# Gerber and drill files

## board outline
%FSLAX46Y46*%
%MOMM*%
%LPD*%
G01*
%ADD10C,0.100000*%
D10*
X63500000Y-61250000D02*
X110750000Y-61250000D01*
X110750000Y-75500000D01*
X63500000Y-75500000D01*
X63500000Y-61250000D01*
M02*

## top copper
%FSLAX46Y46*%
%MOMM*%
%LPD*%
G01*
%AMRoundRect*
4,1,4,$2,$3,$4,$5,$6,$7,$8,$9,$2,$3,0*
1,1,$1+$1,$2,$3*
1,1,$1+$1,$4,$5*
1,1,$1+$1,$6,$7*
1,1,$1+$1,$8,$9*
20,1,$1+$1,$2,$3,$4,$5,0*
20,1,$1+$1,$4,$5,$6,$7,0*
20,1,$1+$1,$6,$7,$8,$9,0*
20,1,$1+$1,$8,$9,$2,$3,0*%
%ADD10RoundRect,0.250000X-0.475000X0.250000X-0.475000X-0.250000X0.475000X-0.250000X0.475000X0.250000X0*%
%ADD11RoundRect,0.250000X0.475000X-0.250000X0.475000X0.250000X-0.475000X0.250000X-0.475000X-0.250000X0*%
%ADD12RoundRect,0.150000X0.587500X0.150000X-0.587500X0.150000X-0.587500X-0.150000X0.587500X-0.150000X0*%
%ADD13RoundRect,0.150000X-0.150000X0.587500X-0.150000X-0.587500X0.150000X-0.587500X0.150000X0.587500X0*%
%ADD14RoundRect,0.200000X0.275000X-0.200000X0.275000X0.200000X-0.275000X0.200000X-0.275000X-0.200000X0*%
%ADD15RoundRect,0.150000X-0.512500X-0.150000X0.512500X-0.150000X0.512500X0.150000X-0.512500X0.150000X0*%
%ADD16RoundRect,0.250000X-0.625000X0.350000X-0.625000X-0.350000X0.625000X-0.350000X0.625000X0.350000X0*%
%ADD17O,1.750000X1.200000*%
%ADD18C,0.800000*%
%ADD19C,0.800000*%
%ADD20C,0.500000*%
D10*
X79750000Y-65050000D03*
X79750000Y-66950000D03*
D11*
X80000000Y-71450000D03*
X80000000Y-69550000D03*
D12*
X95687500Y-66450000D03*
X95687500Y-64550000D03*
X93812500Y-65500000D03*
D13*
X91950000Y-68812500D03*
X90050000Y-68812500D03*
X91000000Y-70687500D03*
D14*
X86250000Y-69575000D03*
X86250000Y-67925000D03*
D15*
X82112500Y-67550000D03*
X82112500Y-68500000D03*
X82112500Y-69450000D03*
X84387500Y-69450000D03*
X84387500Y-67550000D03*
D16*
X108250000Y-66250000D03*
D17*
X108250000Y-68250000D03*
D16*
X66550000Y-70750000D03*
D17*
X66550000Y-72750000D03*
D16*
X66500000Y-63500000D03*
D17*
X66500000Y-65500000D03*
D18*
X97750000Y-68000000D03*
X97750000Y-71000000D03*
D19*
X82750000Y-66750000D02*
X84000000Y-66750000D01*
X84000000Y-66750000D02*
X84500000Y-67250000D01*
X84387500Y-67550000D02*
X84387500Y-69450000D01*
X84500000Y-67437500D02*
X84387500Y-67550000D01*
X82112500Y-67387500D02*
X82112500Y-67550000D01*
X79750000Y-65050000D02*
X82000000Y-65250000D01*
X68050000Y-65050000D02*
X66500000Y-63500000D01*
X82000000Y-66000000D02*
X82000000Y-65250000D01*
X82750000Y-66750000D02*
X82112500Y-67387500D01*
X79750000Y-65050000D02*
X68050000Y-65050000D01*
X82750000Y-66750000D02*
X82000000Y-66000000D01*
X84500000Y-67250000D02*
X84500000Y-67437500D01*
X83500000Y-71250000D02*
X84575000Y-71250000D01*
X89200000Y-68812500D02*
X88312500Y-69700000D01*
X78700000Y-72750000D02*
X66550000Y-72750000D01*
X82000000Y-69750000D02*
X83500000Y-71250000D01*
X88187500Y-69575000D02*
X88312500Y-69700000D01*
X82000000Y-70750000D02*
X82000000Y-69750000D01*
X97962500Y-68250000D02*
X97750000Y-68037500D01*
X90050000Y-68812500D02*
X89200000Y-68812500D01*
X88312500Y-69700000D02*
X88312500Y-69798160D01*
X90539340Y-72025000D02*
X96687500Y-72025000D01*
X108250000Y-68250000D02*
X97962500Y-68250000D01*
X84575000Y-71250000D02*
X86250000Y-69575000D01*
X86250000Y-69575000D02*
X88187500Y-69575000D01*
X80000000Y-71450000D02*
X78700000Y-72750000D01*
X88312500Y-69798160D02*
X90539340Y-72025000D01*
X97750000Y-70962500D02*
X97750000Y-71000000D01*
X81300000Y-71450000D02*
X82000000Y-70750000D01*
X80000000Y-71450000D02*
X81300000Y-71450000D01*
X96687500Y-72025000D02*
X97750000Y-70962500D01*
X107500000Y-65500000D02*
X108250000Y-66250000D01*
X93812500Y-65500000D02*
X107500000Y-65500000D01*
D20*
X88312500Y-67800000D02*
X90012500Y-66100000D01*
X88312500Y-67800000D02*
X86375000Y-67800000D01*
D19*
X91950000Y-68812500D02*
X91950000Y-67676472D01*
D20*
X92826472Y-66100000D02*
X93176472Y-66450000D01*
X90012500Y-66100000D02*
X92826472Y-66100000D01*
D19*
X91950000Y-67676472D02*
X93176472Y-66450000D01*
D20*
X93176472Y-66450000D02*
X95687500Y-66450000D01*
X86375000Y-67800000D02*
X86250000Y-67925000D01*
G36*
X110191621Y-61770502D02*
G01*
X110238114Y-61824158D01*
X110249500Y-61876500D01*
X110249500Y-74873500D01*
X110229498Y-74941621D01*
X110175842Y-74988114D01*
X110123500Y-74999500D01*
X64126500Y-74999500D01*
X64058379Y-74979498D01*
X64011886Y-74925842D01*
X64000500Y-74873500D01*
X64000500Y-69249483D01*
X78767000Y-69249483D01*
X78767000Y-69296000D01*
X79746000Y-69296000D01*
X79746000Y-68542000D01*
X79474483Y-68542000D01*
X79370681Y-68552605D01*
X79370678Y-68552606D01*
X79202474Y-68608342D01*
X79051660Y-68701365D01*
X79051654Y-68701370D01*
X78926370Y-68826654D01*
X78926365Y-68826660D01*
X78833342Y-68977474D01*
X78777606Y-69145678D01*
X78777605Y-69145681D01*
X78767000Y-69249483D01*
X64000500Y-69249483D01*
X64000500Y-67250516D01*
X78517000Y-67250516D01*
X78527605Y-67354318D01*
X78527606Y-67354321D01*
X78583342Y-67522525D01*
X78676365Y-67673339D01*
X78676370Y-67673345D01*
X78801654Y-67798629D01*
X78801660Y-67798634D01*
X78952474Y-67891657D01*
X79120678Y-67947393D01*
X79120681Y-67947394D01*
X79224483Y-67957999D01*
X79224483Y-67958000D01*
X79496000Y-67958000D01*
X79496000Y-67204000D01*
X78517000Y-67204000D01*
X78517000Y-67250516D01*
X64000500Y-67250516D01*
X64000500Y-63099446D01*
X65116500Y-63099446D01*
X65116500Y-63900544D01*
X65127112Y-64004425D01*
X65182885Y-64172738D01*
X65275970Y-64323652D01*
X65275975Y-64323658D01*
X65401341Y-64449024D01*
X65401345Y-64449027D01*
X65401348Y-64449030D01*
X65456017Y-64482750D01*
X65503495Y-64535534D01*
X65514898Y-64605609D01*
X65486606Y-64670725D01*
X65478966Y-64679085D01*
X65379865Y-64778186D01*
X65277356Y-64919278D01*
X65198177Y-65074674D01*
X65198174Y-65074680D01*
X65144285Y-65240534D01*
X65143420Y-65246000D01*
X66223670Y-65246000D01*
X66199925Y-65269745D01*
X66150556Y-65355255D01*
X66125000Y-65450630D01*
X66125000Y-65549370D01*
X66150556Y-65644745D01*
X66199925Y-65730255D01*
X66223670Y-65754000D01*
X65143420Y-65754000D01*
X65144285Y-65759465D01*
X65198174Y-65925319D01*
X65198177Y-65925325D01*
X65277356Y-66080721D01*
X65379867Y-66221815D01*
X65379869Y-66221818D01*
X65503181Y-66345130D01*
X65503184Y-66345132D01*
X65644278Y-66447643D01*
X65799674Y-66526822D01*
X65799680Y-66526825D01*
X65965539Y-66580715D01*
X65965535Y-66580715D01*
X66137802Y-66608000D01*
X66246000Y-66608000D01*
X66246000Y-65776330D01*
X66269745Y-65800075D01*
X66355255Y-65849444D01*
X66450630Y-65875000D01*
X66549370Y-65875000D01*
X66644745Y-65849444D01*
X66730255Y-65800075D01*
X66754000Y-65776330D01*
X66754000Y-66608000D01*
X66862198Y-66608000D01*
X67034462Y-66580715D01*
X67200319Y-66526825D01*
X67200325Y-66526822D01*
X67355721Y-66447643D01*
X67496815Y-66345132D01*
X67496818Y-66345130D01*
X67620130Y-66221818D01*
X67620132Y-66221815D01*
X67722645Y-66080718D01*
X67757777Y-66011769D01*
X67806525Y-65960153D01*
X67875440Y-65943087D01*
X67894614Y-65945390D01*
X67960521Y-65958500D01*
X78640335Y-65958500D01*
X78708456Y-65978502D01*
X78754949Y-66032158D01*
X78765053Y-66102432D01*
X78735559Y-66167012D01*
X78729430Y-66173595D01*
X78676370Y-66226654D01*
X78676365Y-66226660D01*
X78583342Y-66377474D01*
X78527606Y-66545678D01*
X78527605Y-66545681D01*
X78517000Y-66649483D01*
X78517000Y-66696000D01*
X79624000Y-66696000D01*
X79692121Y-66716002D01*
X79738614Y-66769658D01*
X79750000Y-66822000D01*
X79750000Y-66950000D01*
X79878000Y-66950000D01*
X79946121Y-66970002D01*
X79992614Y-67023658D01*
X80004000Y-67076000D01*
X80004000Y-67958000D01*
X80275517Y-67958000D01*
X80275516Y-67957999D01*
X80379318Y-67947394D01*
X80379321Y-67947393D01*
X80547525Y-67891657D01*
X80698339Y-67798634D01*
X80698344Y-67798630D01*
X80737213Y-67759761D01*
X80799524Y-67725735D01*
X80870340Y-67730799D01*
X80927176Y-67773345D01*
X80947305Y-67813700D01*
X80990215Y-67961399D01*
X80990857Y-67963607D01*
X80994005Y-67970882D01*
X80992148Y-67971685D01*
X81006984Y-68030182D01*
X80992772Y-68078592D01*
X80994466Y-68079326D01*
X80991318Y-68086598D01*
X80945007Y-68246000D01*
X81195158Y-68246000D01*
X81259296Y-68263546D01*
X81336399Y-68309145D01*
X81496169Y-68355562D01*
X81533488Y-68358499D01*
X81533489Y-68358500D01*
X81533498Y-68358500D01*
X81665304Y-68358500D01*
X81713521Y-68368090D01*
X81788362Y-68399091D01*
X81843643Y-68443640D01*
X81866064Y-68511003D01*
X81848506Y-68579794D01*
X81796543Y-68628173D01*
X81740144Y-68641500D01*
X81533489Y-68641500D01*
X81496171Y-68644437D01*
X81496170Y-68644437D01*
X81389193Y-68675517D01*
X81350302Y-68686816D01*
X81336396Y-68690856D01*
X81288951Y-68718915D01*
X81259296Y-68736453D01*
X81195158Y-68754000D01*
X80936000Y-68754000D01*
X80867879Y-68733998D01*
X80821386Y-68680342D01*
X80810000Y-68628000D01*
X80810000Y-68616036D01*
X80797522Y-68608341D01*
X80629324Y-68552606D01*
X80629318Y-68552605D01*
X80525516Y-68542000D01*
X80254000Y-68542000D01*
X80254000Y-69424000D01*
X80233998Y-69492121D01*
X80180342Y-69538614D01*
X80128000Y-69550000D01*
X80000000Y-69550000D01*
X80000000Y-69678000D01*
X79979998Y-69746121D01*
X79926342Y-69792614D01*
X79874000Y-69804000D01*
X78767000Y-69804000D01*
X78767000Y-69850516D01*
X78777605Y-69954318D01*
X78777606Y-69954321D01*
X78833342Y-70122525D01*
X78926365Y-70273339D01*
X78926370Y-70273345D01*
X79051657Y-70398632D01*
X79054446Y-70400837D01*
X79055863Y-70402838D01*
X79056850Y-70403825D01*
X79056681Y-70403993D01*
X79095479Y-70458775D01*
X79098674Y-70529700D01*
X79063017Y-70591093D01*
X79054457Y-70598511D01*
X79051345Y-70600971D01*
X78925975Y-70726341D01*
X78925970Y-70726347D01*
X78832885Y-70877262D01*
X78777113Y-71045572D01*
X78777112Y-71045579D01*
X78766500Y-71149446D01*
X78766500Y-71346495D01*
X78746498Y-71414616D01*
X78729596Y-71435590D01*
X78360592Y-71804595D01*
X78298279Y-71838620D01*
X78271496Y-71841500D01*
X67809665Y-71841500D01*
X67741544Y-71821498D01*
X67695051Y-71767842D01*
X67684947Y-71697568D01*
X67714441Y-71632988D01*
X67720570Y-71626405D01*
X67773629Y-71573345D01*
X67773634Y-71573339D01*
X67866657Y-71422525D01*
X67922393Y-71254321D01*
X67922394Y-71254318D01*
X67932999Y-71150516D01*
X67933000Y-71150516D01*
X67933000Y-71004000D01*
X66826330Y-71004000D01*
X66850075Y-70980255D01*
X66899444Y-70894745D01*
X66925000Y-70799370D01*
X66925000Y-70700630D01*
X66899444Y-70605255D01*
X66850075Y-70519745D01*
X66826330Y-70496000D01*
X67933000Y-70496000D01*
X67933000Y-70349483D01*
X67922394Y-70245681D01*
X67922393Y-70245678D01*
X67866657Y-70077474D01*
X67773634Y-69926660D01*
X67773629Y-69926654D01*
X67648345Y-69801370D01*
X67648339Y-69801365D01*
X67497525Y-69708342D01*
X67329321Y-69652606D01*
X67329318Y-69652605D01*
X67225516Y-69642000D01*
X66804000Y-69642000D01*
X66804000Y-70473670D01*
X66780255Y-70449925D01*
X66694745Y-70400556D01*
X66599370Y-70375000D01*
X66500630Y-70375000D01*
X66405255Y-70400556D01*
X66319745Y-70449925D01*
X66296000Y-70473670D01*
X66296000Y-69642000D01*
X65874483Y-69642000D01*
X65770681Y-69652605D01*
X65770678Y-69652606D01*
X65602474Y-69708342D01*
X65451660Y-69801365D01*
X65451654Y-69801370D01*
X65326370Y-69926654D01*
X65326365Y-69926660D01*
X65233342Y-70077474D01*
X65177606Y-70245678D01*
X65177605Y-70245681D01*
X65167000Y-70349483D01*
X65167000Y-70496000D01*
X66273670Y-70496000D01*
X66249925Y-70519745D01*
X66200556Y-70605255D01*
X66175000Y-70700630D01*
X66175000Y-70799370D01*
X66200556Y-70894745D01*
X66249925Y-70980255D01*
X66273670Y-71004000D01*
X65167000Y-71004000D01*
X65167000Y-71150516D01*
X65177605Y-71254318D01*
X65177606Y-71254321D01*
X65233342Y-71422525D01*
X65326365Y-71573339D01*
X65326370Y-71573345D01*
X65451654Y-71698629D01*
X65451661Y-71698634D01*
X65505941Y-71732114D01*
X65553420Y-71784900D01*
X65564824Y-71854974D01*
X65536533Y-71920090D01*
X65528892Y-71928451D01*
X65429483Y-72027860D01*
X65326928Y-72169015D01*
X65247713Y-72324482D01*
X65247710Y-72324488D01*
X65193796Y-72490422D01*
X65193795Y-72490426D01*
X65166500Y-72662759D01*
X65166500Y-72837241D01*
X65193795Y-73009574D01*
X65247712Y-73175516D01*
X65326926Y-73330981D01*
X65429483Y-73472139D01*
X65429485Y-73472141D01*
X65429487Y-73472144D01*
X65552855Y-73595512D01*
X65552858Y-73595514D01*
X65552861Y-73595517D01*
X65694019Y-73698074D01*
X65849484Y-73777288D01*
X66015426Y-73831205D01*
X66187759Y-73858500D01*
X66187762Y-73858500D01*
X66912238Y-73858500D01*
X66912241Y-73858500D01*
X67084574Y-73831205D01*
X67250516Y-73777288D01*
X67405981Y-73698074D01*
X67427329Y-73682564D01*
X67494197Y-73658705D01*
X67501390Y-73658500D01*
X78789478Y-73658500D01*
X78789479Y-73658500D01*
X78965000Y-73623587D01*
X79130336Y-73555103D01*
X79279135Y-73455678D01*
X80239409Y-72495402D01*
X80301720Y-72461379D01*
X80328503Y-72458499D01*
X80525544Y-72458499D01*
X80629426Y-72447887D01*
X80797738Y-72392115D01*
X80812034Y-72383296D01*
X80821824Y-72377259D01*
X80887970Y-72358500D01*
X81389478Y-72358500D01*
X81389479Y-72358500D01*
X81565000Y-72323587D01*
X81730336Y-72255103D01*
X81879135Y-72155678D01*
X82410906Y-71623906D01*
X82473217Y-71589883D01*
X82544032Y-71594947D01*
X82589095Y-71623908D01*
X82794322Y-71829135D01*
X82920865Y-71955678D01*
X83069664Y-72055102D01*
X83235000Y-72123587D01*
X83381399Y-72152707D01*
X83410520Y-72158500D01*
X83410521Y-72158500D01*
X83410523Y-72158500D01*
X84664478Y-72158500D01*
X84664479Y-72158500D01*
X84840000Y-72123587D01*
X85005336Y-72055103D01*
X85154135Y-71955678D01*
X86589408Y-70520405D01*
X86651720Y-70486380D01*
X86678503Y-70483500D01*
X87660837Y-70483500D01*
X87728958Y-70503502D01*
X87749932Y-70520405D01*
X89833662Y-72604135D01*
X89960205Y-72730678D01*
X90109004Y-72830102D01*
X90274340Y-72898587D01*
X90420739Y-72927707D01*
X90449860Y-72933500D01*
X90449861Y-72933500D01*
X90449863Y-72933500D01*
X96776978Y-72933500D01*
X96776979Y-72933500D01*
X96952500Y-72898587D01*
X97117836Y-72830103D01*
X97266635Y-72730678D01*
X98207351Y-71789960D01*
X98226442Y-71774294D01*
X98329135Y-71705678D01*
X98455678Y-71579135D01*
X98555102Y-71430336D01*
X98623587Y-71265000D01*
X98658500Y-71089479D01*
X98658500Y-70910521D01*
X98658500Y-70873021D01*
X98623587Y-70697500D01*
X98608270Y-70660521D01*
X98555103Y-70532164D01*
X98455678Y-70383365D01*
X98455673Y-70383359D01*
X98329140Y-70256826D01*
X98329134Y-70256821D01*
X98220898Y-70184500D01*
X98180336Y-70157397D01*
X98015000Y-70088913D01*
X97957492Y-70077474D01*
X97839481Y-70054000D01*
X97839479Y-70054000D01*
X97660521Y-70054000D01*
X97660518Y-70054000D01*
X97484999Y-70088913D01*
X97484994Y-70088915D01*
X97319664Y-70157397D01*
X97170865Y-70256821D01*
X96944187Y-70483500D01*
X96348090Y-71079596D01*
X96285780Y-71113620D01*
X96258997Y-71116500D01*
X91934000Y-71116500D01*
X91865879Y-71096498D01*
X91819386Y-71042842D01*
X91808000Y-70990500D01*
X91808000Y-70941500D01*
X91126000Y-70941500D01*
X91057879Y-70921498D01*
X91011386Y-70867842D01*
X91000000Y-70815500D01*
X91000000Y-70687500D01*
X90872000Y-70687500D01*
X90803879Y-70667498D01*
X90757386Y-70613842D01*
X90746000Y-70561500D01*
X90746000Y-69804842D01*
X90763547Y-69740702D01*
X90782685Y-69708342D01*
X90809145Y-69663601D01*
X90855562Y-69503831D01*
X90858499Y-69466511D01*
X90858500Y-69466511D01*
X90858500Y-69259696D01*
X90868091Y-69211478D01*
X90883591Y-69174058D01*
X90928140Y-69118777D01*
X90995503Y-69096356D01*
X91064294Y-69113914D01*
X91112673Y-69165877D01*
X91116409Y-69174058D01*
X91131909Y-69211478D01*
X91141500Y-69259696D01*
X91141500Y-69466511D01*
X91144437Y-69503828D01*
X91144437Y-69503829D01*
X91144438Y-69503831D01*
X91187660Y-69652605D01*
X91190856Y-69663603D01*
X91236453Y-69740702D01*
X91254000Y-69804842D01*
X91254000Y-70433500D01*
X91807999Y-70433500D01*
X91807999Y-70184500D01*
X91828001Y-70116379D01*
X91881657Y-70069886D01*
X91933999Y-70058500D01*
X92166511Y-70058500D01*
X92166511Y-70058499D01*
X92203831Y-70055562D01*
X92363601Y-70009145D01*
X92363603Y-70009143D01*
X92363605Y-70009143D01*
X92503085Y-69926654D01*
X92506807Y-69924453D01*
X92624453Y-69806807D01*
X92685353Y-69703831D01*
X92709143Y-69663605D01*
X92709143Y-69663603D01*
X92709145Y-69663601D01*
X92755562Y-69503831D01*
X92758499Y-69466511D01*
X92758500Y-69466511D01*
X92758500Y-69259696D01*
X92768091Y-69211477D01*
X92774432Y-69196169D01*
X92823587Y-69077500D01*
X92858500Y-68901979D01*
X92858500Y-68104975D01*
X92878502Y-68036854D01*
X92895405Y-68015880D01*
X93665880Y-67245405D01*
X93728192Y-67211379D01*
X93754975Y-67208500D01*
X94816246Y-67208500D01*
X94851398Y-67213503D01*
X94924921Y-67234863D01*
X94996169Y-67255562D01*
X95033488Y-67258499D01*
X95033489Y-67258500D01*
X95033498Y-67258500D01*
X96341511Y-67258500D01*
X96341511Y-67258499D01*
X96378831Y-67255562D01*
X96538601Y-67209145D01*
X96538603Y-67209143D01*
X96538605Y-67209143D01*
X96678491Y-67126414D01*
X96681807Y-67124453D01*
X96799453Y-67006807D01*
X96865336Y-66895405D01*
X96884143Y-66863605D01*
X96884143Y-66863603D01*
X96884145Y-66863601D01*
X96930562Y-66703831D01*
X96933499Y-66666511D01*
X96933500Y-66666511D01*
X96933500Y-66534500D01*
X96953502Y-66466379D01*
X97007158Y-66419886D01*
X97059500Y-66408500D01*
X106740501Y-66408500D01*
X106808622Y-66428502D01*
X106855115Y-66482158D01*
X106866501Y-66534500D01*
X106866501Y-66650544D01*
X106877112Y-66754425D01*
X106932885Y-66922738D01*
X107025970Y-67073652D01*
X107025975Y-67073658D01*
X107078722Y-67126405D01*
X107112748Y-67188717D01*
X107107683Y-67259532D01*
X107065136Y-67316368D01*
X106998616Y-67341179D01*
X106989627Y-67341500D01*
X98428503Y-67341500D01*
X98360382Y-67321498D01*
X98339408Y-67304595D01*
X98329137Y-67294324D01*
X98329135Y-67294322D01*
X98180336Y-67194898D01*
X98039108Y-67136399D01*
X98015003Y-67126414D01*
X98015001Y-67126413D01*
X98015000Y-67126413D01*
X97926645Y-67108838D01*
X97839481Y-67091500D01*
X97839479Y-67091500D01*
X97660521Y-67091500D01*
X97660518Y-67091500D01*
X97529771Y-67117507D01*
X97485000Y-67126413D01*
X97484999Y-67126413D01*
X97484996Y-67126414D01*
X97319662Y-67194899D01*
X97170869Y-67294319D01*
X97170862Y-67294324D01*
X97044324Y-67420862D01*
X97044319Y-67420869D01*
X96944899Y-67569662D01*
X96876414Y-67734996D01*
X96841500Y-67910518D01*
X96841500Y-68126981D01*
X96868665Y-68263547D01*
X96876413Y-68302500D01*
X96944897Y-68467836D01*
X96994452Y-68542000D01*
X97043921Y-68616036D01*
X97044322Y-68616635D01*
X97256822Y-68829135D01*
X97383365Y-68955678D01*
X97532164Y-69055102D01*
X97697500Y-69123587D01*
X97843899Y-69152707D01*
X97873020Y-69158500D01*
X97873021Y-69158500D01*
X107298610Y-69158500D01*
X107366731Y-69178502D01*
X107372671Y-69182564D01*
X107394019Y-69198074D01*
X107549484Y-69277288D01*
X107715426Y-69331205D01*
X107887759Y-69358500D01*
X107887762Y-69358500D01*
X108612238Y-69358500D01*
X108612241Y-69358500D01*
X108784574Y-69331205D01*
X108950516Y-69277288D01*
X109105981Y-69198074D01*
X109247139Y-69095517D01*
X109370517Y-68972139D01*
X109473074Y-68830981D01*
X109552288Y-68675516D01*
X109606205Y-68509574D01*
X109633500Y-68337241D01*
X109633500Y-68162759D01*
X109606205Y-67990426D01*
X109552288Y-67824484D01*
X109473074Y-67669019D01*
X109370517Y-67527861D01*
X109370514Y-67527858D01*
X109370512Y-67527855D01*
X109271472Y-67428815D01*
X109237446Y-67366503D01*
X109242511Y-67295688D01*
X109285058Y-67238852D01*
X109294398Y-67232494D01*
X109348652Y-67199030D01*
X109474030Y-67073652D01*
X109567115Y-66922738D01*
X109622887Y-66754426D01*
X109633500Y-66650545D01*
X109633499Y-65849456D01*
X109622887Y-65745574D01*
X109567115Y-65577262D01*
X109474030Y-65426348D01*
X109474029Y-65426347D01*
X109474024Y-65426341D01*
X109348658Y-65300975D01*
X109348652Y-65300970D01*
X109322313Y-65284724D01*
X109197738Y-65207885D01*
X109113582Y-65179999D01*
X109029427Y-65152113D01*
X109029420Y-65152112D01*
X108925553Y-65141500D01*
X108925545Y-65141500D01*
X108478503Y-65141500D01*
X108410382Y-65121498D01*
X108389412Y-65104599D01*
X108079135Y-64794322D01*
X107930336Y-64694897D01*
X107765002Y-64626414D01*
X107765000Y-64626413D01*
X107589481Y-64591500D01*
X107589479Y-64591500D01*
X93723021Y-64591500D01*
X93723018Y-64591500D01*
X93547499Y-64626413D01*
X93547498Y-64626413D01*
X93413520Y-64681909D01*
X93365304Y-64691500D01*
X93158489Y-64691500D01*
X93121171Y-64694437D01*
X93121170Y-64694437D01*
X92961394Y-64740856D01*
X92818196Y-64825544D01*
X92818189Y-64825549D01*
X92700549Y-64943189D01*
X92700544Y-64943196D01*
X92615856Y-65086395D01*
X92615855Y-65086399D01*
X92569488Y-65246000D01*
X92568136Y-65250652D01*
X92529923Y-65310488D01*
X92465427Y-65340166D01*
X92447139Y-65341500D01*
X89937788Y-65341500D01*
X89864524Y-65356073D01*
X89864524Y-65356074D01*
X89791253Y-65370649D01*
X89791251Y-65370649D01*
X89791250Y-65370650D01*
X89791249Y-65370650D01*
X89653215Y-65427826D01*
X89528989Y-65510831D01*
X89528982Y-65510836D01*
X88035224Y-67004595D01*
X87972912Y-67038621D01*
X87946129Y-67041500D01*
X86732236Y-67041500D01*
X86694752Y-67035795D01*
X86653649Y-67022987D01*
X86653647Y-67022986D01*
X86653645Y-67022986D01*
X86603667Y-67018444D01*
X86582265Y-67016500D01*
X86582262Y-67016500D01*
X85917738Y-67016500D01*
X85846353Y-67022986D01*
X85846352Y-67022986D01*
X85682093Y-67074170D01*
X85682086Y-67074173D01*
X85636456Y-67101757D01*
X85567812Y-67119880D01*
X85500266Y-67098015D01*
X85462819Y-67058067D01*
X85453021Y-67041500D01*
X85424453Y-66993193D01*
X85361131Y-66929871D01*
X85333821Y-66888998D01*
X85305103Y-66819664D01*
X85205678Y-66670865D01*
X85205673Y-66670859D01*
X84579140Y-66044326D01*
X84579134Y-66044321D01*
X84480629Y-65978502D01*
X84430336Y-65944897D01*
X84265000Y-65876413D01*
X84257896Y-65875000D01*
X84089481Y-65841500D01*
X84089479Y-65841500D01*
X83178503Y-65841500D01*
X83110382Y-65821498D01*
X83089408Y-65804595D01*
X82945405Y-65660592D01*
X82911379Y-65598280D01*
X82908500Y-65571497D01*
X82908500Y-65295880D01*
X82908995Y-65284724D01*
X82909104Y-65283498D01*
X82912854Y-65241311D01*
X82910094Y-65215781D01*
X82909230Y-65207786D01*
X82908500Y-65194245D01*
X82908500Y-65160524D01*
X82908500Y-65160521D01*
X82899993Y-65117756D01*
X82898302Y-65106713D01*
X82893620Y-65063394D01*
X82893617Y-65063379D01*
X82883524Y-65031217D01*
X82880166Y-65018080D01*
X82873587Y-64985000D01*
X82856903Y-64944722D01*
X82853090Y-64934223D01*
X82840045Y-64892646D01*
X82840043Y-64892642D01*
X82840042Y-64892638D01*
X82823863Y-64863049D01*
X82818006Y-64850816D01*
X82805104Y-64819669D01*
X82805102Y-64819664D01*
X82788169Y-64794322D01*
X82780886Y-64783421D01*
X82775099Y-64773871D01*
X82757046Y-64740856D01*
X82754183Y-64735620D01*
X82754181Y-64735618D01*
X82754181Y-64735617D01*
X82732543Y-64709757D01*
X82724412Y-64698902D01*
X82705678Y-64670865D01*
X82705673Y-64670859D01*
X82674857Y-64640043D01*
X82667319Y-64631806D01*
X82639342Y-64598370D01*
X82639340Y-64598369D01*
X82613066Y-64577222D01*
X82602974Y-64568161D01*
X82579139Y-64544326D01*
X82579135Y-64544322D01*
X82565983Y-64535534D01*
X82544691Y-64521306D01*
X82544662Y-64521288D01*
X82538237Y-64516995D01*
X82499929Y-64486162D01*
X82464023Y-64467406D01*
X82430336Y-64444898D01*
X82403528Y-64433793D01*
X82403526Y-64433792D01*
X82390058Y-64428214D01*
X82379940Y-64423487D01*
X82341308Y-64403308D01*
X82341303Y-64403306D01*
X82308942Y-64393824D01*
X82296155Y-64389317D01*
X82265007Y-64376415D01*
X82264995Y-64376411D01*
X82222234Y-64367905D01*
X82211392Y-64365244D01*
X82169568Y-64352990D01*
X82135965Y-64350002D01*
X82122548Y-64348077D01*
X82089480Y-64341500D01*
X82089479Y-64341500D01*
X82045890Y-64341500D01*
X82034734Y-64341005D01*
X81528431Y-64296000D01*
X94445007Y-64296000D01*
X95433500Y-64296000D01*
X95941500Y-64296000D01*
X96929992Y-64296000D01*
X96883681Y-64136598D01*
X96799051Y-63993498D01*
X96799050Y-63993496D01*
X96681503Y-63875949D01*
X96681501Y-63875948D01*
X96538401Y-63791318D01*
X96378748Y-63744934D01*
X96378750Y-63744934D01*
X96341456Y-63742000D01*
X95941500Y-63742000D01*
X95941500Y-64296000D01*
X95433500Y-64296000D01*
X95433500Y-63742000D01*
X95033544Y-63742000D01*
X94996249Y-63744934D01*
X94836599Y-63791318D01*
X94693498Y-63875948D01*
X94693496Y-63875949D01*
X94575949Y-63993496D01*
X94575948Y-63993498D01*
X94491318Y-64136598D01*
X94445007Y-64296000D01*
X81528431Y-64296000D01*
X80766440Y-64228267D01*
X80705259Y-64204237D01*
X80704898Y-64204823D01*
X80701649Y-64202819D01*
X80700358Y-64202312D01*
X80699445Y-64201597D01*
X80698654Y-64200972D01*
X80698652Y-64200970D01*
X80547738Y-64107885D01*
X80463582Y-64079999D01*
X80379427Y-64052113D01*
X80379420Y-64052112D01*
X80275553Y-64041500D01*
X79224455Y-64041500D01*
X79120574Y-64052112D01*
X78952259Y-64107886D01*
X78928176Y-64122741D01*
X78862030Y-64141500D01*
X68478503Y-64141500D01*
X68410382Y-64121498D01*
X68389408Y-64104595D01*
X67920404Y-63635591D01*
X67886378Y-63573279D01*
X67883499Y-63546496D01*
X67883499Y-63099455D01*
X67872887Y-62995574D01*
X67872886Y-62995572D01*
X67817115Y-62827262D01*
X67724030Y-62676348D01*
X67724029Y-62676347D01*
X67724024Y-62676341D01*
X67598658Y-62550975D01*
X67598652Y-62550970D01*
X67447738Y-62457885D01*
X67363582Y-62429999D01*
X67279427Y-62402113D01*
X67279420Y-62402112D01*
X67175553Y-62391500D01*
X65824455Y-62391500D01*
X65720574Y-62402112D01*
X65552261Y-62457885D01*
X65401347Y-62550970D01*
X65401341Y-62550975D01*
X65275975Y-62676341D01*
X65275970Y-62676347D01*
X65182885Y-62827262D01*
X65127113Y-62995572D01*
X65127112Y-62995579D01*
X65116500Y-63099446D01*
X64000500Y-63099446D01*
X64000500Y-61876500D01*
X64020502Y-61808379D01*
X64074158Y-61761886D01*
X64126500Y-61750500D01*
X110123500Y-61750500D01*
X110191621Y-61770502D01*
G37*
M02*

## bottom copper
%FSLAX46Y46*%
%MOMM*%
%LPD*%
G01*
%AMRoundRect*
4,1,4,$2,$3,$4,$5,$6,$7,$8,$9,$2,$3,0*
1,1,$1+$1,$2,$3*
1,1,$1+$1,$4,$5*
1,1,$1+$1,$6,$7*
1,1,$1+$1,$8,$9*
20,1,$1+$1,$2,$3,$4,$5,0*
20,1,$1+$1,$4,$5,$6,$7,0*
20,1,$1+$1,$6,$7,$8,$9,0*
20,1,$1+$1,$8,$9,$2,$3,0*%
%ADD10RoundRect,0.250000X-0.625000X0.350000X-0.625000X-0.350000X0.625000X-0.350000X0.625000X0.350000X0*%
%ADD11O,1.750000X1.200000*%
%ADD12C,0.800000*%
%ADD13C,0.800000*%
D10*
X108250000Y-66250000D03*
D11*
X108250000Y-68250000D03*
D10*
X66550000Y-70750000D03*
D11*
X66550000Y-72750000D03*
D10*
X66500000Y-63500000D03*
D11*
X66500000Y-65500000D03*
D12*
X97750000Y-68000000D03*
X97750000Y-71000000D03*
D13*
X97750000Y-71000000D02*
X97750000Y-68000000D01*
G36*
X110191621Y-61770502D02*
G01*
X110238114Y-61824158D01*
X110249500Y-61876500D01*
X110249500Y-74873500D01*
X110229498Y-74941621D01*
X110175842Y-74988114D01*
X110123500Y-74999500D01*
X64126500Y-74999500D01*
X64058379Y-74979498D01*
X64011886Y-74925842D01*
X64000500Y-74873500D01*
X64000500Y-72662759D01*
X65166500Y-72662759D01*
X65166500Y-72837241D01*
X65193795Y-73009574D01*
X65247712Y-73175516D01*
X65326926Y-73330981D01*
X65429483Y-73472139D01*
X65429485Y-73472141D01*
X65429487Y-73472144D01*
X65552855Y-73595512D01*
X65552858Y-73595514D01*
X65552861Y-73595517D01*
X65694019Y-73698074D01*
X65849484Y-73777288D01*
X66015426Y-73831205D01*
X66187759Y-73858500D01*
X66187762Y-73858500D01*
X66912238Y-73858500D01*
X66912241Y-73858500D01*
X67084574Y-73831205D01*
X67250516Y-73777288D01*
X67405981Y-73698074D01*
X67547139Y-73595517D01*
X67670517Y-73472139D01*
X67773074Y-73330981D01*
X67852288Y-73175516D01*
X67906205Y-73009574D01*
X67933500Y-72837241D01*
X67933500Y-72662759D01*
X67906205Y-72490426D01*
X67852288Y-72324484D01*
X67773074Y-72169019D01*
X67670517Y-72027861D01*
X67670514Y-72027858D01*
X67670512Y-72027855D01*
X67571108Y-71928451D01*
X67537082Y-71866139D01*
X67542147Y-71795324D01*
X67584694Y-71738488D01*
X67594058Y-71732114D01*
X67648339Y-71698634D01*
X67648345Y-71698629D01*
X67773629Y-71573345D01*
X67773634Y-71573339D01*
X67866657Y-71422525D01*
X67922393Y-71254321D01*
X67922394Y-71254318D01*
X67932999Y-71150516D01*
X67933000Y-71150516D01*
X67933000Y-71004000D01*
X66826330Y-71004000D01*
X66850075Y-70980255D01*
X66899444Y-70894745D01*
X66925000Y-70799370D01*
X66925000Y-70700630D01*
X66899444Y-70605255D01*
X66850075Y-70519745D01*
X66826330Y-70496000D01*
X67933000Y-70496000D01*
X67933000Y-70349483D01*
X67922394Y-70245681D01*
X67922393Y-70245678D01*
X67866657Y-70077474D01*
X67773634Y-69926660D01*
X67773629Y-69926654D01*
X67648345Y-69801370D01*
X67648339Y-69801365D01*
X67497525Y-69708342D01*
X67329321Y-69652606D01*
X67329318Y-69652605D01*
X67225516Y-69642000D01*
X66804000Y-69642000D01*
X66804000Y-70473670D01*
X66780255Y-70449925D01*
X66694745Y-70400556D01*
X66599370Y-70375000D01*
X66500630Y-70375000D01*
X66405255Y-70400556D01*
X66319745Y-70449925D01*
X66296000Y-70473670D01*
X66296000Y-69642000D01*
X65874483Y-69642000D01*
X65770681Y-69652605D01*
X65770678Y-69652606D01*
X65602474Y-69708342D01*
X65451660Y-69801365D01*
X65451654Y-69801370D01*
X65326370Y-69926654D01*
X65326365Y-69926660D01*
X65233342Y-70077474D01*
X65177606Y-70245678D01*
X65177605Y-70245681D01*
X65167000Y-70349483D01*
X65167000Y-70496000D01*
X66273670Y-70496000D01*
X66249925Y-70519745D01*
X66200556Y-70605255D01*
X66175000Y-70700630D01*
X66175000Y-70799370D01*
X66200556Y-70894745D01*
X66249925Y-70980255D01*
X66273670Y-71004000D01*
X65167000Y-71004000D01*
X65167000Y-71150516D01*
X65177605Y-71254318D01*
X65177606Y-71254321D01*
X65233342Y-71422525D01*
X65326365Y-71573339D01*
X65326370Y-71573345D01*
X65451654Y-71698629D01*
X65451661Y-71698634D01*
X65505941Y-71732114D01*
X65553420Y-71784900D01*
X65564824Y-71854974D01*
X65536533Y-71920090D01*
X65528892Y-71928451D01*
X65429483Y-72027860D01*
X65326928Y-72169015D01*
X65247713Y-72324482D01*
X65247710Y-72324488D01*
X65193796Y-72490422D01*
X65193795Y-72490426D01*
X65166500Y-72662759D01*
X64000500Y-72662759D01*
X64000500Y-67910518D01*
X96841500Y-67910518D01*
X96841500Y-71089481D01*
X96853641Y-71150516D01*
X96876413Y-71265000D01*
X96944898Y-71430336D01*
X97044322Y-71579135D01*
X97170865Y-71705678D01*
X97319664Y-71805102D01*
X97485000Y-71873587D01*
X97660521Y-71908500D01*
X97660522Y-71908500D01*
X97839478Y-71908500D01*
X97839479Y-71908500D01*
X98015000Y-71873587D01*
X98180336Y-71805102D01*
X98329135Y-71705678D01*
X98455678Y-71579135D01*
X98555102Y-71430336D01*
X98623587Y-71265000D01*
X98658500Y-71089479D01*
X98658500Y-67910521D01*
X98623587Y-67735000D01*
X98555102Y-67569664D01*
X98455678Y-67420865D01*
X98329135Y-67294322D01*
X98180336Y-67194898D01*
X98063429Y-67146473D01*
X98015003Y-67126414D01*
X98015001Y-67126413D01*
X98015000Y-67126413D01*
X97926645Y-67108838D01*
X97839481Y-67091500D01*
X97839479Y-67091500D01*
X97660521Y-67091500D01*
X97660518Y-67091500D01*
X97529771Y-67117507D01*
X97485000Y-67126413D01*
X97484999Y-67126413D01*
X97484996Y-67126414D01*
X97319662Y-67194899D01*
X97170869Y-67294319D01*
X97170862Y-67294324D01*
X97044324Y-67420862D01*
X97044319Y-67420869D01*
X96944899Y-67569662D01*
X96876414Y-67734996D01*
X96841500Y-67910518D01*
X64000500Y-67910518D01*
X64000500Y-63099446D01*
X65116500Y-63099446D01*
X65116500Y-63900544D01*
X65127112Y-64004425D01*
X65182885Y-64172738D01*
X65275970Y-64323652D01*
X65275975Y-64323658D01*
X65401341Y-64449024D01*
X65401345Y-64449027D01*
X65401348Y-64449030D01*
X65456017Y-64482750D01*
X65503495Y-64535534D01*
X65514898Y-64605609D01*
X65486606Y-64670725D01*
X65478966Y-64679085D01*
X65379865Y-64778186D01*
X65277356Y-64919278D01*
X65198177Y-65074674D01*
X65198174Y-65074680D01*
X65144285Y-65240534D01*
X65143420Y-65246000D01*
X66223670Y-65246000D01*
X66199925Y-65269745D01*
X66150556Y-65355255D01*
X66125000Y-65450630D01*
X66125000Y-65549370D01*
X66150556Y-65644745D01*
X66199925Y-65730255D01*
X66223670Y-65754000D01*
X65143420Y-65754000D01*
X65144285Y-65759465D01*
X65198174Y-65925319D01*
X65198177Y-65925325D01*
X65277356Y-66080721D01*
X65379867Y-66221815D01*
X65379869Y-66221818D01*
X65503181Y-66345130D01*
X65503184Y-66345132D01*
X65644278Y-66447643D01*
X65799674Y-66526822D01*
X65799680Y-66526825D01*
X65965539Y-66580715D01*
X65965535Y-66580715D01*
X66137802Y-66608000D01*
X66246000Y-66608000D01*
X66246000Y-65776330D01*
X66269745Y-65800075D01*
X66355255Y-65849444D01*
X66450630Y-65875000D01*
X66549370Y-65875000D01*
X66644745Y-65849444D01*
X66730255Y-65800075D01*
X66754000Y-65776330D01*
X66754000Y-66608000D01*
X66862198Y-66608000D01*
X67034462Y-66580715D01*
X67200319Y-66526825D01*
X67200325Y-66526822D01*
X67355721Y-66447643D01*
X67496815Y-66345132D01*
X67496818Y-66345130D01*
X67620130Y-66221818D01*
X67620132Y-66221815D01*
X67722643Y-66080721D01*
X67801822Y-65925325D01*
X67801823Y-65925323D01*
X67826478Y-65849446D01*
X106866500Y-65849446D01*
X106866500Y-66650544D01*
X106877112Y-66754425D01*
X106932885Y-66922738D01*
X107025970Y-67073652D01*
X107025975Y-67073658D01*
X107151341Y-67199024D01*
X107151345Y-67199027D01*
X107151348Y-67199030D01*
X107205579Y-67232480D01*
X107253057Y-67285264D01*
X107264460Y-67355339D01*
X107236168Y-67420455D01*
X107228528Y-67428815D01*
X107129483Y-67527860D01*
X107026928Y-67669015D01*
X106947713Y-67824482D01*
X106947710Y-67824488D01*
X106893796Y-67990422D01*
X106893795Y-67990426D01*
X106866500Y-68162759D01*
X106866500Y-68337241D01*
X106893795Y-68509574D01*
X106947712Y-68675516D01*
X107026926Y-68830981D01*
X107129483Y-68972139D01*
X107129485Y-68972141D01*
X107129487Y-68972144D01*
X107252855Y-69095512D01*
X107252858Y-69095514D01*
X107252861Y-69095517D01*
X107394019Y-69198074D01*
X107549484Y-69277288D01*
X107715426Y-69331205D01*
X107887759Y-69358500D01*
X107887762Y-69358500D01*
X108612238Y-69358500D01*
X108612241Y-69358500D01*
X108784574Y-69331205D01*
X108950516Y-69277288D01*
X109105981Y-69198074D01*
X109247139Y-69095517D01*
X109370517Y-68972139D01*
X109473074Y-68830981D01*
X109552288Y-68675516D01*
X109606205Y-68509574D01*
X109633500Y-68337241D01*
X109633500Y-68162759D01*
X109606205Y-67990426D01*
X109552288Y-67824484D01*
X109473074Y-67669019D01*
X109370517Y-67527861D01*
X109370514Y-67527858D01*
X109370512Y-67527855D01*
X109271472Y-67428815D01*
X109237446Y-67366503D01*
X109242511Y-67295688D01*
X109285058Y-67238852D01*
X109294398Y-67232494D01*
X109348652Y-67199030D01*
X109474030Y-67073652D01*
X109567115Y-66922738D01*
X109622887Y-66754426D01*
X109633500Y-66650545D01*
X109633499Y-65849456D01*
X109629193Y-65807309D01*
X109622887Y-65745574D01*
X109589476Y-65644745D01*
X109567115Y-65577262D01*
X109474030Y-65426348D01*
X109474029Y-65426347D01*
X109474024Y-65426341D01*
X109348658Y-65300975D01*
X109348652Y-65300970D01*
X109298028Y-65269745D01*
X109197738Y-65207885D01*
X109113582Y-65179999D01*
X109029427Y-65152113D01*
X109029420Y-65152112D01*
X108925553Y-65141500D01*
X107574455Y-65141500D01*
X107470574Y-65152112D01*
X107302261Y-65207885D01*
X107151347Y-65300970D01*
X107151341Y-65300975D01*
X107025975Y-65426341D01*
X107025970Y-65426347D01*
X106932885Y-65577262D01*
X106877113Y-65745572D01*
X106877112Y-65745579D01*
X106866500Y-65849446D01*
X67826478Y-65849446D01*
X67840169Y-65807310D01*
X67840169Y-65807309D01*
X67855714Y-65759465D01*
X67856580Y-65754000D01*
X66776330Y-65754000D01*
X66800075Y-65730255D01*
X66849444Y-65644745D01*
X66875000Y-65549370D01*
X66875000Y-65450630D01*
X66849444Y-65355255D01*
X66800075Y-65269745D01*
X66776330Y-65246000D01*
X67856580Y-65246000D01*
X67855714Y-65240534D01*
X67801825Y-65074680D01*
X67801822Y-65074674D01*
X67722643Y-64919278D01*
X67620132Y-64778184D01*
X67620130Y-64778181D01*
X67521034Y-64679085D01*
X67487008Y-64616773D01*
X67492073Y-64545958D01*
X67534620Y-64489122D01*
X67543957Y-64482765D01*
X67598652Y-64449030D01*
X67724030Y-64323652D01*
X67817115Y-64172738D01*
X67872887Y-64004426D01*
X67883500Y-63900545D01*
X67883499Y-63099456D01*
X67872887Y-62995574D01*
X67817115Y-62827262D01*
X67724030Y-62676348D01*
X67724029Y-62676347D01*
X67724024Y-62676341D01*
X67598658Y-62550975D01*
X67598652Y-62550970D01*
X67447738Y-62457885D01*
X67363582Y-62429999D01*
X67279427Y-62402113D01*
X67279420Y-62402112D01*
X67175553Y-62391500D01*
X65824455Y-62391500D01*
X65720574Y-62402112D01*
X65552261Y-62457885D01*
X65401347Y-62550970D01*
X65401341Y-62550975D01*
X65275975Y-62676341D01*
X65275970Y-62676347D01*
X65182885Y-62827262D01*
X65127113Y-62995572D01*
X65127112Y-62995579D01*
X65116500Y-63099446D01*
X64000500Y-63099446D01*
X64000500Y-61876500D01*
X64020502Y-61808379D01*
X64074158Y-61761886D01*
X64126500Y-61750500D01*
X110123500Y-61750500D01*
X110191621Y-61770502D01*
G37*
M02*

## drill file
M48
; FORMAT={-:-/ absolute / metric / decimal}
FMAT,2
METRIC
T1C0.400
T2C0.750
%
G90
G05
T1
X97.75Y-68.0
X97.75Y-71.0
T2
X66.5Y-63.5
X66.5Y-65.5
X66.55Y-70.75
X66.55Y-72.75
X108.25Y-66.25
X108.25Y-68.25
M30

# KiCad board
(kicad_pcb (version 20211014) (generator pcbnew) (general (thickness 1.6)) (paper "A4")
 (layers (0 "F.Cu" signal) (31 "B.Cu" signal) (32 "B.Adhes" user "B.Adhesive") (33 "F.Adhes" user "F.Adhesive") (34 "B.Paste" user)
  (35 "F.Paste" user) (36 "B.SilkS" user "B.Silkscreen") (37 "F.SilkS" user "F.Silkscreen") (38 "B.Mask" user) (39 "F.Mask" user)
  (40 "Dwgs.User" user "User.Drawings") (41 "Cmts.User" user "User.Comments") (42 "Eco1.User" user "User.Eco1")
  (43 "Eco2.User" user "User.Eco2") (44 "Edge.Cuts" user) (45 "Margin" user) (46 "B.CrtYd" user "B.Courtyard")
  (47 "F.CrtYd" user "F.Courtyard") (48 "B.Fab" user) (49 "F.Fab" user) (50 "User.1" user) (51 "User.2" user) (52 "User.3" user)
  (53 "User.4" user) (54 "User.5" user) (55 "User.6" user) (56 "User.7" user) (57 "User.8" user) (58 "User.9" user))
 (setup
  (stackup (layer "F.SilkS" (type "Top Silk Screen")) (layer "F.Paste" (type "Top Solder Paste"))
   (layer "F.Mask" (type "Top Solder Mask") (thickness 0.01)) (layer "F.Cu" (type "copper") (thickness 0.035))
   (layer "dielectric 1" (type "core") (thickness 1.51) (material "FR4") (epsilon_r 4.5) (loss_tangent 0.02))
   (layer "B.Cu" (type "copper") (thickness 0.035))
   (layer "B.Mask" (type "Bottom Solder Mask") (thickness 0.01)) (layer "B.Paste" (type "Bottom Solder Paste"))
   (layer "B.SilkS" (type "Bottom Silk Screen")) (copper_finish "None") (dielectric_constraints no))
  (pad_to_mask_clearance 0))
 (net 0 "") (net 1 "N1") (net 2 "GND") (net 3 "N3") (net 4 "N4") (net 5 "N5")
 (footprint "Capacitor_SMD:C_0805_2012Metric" (layer "F.Cu") (at 79.75 66 -90)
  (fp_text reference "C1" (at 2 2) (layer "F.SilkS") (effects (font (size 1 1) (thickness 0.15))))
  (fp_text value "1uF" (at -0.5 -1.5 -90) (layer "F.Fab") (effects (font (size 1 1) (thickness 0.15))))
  (pad "1" smd roundrect (at -0.95 0 270) (size 1 1.45) (layers "F.Cu" "F.Paste" "F.Mask") (roundrect_rratio 0.25) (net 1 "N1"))
  (pad "2" smd roundrect (at 0.95 0 270) (size 1 1.45) (layers "F.Cu" "F.Paste" "F.Mask") (roundrect_rratio 0.25) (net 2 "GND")))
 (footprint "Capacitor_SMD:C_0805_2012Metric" (layer "F.Cu") (at 80 70.5 90)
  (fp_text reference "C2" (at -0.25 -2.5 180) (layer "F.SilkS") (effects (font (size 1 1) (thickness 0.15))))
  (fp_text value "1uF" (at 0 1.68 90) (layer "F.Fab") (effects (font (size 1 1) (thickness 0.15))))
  (pad "1" smd roundrect (at -0.95 0 90) (size 1 1.45) (layers "F.Cu" "F.Paste" "F.Mask") (roundrect_rratio 0.25) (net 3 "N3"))
  (pad "2" smd roundrect (at 0.95 0 90) (size 1 1.45) (layers "F.Cu" "F.Paste" "F.Mask") (roundrect_rratio 0.25) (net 2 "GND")))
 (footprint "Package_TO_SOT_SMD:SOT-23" (layer "F.Cu") (at 94.75 65.5 180)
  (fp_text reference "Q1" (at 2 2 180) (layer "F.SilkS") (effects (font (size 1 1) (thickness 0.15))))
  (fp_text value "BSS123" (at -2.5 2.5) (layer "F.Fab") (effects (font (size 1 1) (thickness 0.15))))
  (pad "1" smd roundrect (at -0.9375 -0.95 180) (size 1.475 0.6) (layers "F.Cu" "F.Paste" "F.Mask") (roundrect_rratio 0.25) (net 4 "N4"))
  (pad "2" smd roundrect (at -0.9375 0.95 180) (size 1.475 0.6) (layers "F.Cu" "F.Paste" "F.Mask") (roundrect_rratio 0.25) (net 2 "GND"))
  (pad "3" smd roundrect (at 0.9375 0 180) (size 1.475 0.6) (layers "F.Cu" "F.Paste" "F.Mask") (roundrect_rratio 0.25) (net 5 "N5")))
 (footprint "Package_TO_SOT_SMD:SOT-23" (layer "F.Cu") (at 91 69.75 -90)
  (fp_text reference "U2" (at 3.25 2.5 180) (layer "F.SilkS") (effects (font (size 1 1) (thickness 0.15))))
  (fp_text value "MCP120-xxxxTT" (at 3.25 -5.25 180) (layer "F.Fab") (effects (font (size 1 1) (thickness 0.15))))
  (pad "1" smd roundrect (at -0.9375 -0.95 270) (size 1.475 0.6) (layers "F.Cu" "F.Paste" "F.Mask") (roundrect_rratio 0.25) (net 4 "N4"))
  (pad "2" smd roundrect (at -0.9375 0.95 270) (size 1.475 0.6) (layers "F.Cu" "F.Paste" "F.Mask") (roundrect_rratio 0.25) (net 3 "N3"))
  (pad "3" smd roundrect (at 0.9375 0 270) (size 1.475 0.6) (layers "F.Cu" "F.Paste" "F.Mask") (roundrect_rratio 0.25) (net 2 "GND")))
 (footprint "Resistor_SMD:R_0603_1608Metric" (layer "F.Cu") (at 86.25 68.75 90)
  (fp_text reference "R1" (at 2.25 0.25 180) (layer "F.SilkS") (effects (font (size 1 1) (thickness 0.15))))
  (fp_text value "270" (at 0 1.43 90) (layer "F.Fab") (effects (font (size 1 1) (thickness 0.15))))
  (pad "1" smd roundrect (at -0.825 0 90) (size 0.8 0.95) (layers "F.Cu" "F.Paste" "F.Mask") (roundrect_rratio 0.25) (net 3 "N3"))
  (pad "2" smd roundrect (at 0.825 0 90) (size 0.8 0.95) (layers "F.Cu" "F.Paste" "F.Mask") (roundrect_rratio 0.25) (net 4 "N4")))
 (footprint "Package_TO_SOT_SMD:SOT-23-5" (layer "F.Cu") (at 83.25 68.5)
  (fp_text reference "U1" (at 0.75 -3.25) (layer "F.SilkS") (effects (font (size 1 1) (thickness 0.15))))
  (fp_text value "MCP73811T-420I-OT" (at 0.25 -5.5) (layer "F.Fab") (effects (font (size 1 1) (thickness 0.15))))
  (pad "1" smd roundrect (at -1.1375 -0.95) (size 1.325 0.6) (layers "F.Cu" "F.Paste" "F.Mask") (roundrect_rratio 0.25) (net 1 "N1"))
  (pad "2" smd roundrect (at -1.1375 0) (size 1.325 0.6) (layers "F.Cu" "F.Paste" "F.Mask") (roundrect_rratio 0.25) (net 2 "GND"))
  (pad "3" smd roundrect (at -1.1375 0.95) (size 1.325 0.6) (layers "F.Cu" "F.Paste" "F.Mask") (roundrect_rratio 0.25) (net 3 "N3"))
  (pad "4" smd roundrect (at 1.1375 0.95) (size 1.325 0.6) (layers "F.Cu" "F.Paste" "F.Mask") (roundrect_rratio 0.25) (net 1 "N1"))
  (pad "5" smd roundrect (at 1.1375 -0.95) (size 1.325 0.6) (layers "F.Cu" "F.Paste" "F.Mask") (roundrect_rratio 0.25) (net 1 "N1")))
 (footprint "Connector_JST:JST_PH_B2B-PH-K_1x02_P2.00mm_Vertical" (layer "B.Cu") (at 108.25 66.25 -90)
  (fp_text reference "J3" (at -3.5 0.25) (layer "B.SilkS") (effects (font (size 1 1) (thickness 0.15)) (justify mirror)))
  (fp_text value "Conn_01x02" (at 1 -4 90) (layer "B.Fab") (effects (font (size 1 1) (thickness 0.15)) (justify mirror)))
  (pad "1" thru_hole roundrect (at 0 0 270) (size 1.2 1.75) (drill 0.75) (layers *.Cu *.Mask) (roundrect_rratio 0.2083333333) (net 5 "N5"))
  (pad "2" thru_hole oval (at 2 0 270) (size 1.2 1.75) (drill 0.75) (layers *.Cu *.Mask) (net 3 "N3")))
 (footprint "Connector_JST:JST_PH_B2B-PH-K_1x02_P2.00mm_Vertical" (layer "B.Cu") (at 66.55 70.75 -90)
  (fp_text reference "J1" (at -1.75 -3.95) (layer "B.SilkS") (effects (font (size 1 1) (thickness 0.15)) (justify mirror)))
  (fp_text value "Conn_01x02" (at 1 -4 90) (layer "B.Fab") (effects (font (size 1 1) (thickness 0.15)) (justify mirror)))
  (pad "1" thru_hole roundrect (at 0 0 270) (size 1.2 1.75) (drill 0.75) (layers *.Cu *.Mask) (roundrect_rratio 0.2083333333) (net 2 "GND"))
  (pad "2" thru_hole oval (at 2 0 270) (size 1.2 1.75) (drill 0.75) (layers *.Cu *.Mask) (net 3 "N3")))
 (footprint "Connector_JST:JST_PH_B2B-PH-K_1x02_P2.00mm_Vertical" (layer "B.Cu") (at 66.5 63.5 -90)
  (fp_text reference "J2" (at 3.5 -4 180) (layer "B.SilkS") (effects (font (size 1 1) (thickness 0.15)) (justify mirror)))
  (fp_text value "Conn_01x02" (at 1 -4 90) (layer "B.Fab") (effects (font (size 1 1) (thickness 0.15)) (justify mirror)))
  (pad "1" thru_hole roundrect (at 0 0 270) (size 1.2 1.75) (drill 0.75) (layers *.Cu *.Mask) (roundrect_rratio 0.2083333333) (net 1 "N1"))
  (pad "2" thru_hole oval (at 2 0 270) (size 1.2 1.75) (drill 0.75) (layers *.Cu *.Mask) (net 2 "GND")))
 (gr_rect (start 63.5 61.25) (end 110.75 75.5) (layer "Edge.Cuts") (width 0.1) (fill none))
 (segment (start 82.75 66.75) (end 84 66.75) (width 0.8) (layer "F.Cu") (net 1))
 (segment (start 84 66.75) (end 84.5 67.25) (width 0.8) (layer "F.Cu") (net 1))
 (segment (start 84.3875 67.55) (end 84.3875 69.45) (width 0.8) (layer "F.Cu") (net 1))
 (segment (start 84.5 67.4375) (end 84.3875 67.55) (width 0.8) (layer "F.Cu") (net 1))
 (segment (start 82.1125 67.3875) (end 82.1125 67.55) (width 0.8) (layer "F.Cu") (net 1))
 (segment (start 79.75 65.05) (end 82 65.25) (width 0.8) (layer "F.Cu") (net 1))
 (segment (start 68.05 65.05) (end 66.5 63.5) (width 0.8) (layer "F.Cu") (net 1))
 (segment (start 82 66) (end 82 65.25) (width 0.8) (layer "F.Cu") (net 1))
 (segment (start 82.75 66.75) (end 82.1125 67.3875) (width 0.8) (layer "F.Cu") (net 1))
 (segment (start 79.75 65.05) (end 68.05 65.05) (width 0.8) (layer "F.Cu") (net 1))
 (segment (start 82.75 66.75) (end 82 66) (width 0.8) (layer "F.Cu") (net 1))
 (segment (start 84.5 67.25) (end 84.5 67.4375) (width 0.8) (layer "F.Cu") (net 1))
 (segment (start 83.5 71.25) (end 84.575 71.25) (width 0.8) (layer "F.Cu") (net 3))
 (segment (start 89.2 68.8125) (end 88.3125 69.7) (width 0.8) (layer "F.Cu") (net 3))
 (segment (start 78.7 72.75) (end 66.55 72.75) (width 0.8) (layer "F.Cu") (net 3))
 (segment (start 82 69.75) (end 83.5 71.25) (width 0.8) (layer "F.Cu") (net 3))
 (segment (start 88.1875 69.575) (end 88.3125 69.7) (width 0.8) (layer "F.Cu") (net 3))
 (segment (start 82 70.75) (end 82 69.75) (width 0.8) (layer "F.Cu") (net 3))
 (segment (start 97.9625 68.25) (end 97.75 68.0375) (width 0.8) (layer "F.Cu") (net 3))
 (segment (start 90.05 68.8125) (end 89.2 68.8125) (width 0.8) (layer "F.Cu") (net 3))
 (segment (start 88.3125 69.7) (end 88.3125 69.79816) (width 0.8) (layer "F.Cu") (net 3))
 (segment (start 90.53934 72.025) (end 96.6875 72.025) (width 0.8) (layer "F.Cu") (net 3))
 (segment (start 108.25 68.25) (end 97.9625 68.25) (width 0.8) (layer "F.Cu") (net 3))
 (segment (start 84.575 71.25) (end 86.25 69.575) (width 0.8) (layer "F.Cu") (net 3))
 (segment (start 86.25 69.575) (end 88.1875 69.575) (width 0.8) (layer "F.Cu") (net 3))
 (segment (start 80 71.45) (end 78.7 72.75) (width 0.8) (layer "F.Cu") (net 3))
 (segment (start 88.3125 69.79816) (end 90.53934 72.025) (width 0.8) (layer "F.Cu") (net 3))
 (segment (start 97.75 70.9625) (end 97.75 71) (width 0.8) (layer "F.Cu") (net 3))
 (segment (start 81.3 71.45) (end 82 70.75) (width 0.8) (layer "F.Cu") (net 3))
 (segment (start 80 71.45) (end 81.3 71.45) (width 0.8) (layer "F.Cu") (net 3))
 (segment (start 96.6875 72.025) (end 97.75 70.9625) (width 0.8) (layer "F.Cu") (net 3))
 (via (at 97.75 68) (size 0.8) (drill 0.4) (layers "F.Cu" "B.Cu") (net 3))
 (via (at 97.75 71) (size 0.8) (drill 0.4) (layers "F.Cu" "B.Cu") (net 3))
 (segment (start 97.75 71) (end 97.75 68) (width 0.8) (layer "B.Cu") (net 3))
 (segment (start 107.5 65.5) (end 108.25 66.25) (width 0.8) (layer "F.Cu") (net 5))
 (segment (start 93.8125 65.5) (end 107.5 65.5) (width 0.8) (layer "F.Cu") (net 5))
 (segment (start 88.3125 67.8) (end 90.0125 66.1) (width 0.5) (layer "F.Cu") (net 4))
 (segment (start 88.3125 67.8) (end 86.375 67.8) (width 0.5) (layer "F.Cu") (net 4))
 (segment (start 91.95 68.8125) (end 91.95 67.676472) (width 0.8) (layer "F.Cu") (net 4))
 (segment (start 92.826472 66.1) (end 93.176472 66.45) (width 0.5) (layer "F.Cu") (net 4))
 (segment (start 90.0125 66.1) (end 92.826472 66.1) (width 0.5) (layer "F.Cu") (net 4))
 (segment (start 91.95 67.676472) (end 93.176472 66.45) (width 0.8) (layer "F.Cu") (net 4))
 (segment (start 93.176472 66.45) (end 95.6875 66.45) (width 0.5) (layer "F.Cu") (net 4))
 (segment (start 86.375 67.8) (end 86.25 67.925) (width 0.5) (layer "F.Cu") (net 4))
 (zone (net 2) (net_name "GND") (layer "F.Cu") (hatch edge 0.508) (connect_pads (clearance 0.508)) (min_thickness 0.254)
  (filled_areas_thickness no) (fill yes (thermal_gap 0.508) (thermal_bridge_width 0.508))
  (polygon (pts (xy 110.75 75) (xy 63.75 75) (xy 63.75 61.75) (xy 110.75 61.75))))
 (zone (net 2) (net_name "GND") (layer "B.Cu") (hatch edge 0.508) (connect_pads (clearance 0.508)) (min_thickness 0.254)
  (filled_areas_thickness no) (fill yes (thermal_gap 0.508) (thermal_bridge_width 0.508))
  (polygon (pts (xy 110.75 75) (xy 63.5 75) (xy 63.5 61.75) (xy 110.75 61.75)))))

